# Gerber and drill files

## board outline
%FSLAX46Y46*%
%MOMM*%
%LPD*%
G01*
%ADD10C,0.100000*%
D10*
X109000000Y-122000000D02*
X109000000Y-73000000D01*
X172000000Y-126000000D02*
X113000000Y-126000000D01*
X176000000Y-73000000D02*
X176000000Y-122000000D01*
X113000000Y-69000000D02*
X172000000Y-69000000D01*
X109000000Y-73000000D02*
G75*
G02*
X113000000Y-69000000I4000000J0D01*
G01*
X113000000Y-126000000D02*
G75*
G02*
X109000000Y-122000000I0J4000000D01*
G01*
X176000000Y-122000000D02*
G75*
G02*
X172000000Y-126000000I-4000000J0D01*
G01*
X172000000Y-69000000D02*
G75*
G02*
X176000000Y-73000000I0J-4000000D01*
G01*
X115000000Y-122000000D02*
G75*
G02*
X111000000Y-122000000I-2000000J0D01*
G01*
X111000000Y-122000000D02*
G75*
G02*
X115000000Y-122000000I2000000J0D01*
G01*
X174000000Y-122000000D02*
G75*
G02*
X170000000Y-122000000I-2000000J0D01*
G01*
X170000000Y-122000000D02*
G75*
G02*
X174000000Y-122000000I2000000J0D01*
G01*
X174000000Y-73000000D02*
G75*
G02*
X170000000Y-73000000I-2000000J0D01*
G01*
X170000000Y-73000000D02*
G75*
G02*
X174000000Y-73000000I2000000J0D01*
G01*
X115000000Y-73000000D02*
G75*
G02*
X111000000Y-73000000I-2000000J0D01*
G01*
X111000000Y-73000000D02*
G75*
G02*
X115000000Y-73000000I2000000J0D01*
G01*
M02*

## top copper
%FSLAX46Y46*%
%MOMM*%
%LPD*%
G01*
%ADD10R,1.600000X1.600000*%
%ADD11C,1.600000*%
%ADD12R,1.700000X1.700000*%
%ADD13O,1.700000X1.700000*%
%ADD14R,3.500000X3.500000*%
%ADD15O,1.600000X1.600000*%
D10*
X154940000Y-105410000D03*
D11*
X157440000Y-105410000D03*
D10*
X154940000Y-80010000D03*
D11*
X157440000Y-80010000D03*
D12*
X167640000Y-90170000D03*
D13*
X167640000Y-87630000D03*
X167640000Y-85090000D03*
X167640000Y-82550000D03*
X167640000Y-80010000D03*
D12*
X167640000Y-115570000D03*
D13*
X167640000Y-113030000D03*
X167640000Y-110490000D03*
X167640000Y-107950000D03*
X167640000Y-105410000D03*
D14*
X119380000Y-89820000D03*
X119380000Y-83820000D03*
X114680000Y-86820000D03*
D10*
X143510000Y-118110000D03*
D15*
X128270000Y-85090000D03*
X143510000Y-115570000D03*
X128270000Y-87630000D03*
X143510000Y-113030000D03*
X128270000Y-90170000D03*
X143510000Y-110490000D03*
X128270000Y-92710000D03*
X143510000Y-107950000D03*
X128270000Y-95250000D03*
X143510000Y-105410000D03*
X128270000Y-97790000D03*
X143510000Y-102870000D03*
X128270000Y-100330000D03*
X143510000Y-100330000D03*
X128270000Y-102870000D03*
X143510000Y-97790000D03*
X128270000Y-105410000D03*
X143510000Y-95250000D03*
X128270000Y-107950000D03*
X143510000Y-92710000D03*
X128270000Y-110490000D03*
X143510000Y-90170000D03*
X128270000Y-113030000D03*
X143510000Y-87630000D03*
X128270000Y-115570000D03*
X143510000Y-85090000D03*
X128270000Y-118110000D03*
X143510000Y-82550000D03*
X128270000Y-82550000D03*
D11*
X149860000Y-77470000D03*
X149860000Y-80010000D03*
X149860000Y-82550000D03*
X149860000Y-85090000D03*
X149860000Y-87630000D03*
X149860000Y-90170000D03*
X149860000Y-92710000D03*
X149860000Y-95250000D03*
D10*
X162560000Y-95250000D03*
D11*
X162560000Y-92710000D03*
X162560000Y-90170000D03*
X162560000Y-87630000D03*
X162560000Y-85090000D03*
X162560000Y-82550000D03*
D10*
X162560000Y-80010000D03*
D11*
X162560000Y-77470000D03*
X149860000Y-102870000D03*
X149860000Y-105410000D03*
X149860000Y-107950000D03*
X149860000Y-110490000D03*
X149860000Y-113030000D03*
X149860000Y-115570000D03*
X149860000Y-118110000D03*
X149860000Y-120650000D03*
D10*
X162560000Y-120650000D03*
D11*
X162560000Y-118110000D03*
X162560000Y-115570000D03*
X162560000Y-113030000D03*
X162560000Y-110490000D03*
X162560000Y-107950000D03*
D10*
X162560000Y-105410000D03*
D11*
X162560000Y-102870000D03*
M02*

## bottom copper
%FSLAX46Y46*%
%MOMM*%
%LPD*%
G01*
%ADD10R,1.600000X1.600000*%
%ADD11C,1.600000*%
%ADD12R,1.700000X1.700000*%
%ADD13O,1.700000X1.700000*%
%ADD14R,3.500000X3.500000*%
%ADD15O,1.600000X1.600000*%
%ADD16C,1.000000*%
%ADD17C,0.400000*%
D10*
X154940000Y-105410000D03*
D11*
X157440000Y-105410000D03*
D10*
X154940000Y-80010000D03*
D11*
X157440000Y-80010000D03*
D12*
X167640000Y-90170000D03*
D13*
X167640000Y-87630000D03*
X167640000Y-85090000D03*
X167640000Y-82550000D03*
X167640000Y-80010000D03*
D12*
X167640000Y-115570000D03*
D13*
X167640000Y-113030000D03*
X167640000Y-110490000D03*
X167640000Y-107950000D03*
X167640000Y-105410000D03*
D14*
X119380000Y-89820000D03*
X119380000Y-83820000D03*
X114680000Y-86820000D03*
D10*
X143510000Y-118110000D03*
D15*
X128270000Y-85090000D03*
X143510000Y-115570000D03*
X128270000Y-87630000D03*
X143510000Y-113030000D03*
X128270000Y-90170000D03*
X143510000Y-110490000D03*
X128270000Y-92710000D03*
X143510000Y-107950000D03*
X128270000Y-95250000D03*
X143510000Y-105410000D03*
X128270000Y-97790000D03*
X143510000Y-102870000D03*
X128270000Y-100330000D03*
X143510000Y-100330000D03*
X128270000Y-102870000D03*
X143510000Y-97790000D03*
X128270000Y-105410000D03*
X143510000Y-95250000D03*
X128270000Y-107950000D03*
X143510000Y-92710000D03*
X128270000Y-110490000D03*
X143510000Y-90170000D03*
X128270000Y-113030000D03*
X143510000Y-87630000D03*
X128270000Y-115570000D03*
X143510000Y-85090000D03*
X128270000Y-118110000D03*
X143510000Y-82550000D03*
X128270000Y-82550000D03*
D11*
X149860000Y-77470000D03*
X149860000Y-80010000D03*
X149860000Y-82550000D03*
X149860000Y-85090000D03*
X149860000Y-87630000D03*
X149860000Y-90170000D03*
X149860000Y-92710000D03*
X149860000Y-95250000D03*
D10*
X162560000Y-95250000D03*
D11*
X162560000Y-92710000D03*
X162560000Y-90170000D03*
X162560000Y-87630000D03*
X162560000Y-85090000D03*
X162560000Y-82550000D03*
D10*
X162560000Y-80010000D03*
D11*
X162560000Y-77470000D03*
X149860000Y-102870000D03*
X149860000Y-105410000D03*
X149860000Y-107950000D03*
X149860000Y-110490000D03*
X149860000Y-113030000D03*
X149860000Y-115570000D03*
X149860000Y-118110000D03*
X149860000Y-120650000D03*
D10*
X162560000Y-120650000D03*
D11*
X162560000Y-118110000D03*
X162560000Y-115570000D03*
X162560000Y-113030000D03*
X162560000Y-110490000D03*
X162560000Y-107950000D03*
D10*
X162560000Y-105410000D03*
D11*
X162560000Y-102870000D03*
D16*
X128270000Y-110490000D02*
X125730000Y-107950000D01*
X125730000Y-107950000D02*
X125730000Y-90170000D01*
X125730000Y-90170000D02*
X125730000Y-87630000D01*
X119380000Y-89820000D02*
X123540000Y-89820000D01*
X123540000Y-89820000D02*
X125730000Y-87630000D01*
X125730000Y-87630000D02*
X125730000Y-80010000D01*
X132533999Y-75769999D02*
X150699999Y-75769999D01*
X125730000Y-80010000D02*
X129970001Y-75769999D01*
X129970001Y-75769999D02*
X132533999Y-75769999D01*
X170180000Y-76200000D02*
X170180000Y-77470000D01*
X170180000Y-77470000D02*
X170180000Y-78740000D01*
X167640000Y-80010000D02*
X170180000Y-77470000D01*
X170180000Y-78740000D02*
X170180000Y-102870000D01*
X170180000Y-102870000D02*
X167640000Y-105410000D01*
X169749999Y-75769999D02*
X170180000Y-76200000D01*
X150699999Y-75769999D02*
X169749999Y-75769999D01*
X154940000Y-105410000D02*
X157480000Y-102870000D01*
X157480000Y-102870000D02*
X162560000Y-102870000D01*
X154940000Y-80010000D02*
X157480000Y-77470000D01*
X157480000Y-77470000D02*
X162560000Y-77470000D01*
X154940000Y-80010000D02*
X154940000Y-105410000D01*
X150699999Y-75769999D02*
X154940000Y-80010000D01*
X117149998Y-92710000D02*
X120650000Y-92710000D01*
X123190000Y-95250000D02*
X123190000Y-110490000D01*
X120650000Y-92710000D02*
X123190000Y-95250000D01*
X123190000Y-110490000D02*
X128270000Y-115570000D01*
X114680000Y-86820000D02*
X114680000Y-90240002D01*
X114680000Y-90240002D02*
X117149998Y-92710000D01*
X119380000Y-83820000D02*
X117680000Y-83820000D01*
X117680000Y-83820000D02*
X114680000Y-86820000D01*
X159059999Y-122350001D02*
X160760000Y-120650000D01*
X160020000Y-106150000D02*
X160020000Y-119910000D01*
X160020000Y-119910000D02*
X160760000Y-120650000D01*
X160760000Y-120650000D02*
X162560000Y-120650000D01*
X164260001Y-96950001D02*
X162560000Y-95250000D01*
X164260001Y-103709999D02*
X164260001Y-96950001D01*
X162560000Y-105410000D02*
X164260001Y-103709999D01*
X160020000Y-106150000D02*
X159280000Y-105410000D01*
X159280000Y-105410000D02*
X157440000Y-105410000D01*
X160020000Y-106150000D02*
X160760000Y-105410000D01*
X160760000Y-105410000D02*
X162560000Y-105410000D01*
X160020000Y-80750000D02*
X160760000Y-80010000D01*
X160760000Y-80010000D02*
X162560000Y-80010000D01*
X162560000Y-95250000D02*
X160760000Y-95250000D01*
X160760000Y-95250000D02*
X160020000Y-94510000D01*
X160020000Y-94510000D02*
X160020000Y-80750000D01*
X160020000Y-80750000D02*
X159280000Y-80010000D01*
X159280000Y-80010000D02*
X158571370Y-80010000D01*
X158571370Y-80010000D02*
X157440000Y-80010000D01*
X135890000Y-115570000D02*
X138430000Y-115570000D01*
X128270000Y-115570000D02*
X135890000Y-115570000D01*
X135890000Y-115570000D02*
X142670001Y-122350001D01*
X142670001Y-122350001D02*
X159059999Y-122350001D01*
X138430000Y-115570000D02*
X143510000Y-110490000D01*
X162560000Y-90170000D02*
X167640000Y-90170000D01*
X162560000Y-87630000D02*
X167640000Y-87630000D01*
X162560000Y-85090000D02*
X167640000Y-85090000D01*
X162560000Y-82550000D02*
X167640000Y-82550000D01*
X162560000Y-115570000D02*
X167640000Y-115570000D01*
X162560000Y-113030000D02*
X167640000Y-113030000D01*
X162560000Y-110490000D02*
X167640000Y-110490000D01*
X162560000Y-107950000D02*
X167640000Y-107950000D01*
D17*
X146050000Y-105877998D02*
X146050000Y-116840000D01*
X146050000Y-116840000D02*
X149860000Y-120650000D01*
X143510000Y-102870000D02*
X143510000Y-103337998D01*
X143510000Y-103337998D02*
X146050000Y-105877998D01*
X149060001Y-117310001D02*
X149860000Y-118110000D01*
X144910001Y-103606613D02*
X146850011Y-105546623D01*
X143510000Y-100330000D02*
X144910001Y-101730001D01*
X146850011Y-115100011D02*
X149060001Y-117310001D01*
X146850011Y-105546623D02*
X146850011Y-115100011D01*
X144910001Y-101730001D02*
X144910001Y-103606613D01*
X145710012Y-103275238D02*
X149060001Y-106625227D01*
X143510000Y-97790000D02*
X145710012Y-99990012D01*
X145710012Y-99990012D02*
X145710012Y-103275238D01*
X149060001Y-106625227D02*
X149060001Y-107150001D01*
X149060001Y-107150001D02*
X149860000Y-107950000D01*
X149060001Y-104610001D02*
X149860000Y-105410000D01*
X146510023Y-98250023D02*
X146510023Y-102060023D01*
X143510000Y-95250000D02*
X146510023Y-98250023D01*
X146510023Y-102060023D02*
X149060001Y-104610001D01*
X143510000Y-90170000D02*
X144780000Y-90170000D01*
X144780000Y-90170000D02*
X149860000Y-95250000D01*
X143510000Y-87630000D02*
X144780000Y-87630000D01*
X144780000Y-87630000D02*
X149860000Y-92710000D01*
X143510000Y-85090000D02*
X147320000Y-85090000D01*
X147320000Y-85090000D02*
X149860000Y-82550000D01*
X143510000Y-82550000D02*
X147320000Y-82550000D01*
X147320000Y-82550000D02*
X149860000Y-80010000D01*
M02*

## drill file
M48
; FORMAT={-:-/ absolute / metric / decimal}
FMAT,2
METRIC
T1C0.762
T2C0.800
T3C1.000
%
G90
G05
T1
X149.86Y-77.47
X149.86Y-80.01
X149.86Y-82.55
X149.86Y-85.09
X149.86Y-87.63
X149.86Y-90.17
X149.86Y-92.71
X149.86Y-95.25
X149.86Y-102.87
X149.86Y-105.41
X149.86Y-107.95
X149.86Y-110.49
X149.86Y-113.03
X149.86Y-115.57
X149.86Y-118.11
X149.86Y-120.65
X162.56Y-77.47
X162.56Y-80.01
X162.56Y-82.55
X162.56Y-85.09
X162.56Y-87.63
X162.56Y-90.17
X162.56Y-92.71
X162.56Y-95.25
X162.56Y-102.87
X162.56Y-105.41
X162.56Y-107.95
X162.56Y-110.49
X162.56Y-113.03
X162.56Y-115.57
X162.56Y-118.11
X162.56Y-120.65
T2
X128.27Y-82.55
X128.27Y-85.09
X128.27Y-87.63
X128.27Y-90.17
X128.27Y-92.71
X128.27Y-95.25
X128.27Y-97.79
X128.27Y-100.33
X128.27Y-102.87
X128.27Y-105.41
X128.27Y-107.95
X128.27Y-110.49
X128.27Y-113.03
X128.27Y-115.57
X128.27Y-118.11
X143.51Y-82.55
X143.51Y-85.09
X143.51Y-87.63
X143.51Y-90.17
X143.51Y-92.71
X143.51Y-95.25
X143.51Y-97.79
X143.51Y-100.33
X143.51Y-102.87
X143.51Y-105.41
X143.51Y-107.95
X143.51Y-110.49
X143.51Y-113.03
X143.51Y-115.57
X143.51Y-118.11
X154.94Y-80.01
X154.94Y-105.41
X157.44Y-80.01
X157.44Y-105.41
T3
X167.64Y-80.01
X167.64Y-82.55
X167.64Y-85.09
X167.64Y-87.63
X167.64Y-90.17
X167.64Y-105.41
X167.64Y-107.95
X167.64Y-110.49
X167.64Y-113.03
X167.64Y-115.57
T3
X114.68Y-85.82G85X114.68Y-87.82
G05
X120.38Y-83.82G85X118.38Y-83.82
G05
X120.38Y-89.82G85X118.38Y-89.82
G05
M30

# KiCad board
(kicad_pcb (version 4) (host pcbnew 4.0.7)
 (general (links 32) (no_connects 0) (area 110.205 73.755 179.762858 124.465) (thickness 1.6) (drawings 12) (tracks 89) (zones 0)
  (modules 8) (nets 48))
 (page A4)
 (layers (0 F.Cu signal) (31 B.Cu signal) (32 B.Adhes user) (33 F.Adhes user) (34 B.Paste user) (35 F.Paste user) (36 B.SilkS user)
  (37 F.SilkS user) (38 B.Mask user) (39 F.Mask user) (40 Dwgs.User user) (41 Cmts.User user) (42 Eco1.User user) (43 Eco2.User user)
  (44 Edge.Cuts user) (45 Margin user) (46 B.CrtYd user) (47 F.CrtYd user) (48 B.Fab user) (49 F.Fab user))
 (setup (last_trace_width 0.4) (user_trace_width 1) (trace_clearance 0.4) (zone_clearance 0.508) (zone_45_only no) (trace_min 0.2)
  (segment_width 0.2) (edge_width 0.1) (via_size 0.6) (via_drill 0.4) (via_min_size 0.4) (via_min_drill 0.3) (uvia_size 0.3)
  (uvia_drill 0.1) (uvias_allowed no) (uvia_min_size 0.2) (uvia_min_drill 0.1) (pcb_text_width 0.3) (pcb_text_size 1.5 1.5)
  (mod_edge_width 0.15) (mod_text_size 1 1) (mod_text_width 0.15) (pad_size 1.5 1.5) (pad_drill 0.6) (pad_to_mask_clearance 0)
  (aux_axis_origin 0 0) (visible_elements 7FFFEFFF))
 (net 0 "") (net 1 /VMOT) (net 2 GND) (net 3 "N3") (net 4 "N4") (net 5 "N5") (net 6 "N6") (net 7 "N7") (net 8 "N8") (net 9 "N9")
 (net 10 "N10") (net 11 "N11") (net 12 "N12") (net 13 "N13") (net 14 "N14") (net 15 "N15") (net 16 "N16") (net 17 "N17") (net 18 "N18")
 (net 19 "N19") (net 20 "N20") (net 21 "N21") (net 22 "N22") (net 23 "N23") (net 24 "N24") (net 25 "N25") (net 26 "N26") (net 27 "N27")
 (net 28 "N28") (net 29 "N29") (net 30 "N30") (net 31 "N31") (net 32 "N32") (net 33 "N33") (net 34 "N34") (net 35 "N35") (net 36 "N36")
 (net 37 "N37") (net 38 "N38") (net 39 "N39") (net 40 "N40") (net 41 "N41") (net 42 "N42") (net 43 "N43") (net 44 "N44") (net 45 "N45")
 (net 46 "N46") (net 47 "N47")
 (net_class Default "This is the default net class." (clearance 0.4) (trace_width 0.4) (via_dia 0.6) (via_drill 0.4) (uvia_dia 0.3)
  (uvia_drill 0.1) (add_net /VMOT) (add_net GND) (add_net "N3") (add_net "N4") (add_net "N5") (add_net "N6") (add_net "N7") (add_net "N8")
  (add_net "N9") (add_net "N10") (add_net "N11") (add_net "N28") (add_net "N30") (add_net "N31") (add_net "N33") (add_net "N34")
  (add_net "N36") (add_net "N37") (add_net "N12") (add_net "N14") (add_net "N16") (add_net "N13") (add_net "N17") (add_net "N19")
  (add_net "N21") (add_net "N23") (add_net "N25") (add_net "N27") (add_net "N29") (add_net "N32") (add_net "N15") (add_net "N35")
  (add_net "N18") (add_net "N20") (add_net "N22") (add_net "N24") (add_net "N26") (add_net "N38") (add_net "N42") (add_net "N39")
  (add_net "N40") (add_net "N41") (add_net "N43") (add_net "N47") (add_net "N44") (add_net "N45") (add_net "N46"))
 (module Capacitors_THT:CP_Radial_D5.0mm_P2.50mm (layer F.Cu) (at 154.94 105.41)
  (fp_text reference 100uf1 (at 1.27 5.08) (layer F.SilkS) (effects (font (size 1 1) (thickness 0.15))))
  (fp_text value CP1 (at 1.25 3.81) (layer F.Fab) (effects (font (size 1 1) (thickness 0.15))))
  (pad 1 thru_hole rect (at 0 0) (size 1.6 1.6) (drill 0.8) (layers *.Cu *.Mask) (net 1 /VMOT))
  (pad 2 thru_hole circle (at 2.5 0) (size 1.6 1.6) (drill 0.8) (layers *.Cu *.Mask) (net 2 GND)))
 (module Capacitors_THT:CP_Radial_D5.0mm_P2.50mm (layer F.Cu) (at 154.94 80.01)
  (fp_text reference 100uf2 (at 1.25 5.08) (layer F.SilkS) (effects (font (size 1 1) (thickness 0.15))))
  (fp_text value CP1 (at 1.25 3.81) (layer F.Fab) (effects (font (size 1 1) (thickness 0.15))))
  (pad 1 thru_hole rect (at 0 0) (size 1.6 1.6) (drill 0.8) (layers *.Cu *.Mask) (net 1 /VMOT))
  (pad 2 thru_hole circle (at 2.5 0) (size 1.6 1.6) (drill 0.8) (layers *.Cu *.Mask) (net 2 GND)))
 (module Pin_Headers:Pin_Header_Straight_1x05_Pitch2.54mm (layer F.Cu) (at 167.64 90.17 180)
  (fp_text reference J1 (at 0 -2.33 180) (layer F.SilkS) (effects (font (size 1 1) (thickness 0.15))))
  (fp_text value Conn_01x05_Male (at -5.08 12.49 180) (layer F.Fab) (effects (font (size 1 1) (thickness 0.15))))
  (pad 1 thru_hole rect (at 0 0 180) (size 1.7 1.7) (drill 1) (layers *.Cu *.Mask) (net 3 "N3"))
  (pad 2 thru_hole oval (at 0 2.54 180) (size 1.7 1.7) (drill 1) (layers *.Cu *.Mask) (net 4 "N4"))
  (pad 3 thru_hole oval (at 0 5.08 180) (size 1.7 1.7) (drill 1) (layers *.Cu *.Mask) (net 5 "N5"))
  (pad 4 thru_hole oval (at 0 7.62 180) (size 1.7 1.7) (drill 1) (layers *.Cu *.Mask) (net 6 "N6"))
  (pad 5 thru_hole oval (at 0 10.16 180) (size 1.7 1.7) (drill 1) (layers *.Cu *.Mask) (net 1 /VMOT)))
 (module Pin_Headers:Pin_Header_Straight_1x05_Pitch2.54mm (layer F.Cu) (at 167.64 115.57 180)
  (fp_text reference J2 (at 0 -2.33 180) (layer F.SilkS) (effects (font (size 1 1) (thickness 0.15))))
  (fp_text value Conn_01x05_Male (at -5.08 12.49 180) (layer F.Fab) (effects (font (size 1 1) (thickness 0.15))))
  (pad 1 thru_hole rect (at 0 0 180) (size 1.7 1.7) (drill 1) (layers *.Cu *.Mask) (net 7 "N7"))
  (pad 2 thru_hole oval (at 0 2.54 180) (size 1.7 1.7) (drill 1) (layers *.Cu *.Mask) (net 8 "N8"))
  (pad 3 thru_hole oval (at 0 5.08 180) (size 1.7 1.7) (drill 1) (layers *.Cu *.Mask) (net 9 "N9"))
  (pad 4 thru_hole oval (at 0 7.62 180) (size 1.7 1.7) (drill 1) (layers *.Cu *.Mask) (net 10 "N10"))
  (pad 5 thru_hole oval (at 0 10.16 180) (size 1.7 1.7) (drill 1) (layers *.Cu *.Mask) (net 1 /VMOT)))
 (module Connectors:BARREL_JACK (layer F.Cu) (at 119.38 89.82 270)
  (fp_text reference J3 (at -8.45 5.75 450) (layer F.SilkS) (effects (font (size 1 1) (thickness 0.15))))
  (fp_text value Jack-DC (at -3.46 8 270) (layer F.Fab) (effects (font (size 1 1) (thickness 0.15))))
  (pad 1 thru_hole rect (at 0 0 270) (size 3.5 3.5) (drill oval 1 3) (layers *.Cu *.Mask) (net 1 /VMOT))
  (pad 2 thru_hole rect (at -6 0 270) (size 3.5 3.5) (drill oval 1 3) (layers *.Cu *.Mask) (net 2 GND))
  (pad 3 thru_hole rect (at -3 4.7 270) (size 3.5 3.5) (drill oval 3 1) (layers *.Cu *.Mask) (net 2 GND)))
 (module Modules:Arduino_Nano (layer F.Cu) (at 143.51 118.11 180)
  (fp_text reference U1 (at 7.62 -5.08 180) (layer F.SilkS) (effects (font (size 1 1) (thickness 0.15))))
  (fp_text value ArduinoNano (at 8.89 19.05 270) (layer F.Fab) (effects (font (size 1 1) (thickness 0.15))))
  (pad 1 thru_hole rect (at 0 0 180) (size 1.6 1.6) (drill 0.8) (layers *.Cu *.Mask) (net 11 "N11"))
  (pad 17 thru_hole oval (at 15.24 33.02 180) (size 1.6 1.6) (drill 0.8) (layers *.Cu *.Mask) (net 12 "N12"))
  (pad 2 thru_hole oval (at 0 2.54 180) (size 1.6 1.6) (drill 0.8) (layers *.Cu *.Mask) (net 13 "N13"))
  (pad 18 thru_hole oval (at 15.24 30.48 180) (size 1.6 1.6) (drill 0.8) (layers *.Cu *.Mask) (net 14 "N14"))
  (pad 3 thru_hole oval (at 0 5.08 180) (size 1.6 1.6) (drill 0.8) (layers *.Cu *.Mask) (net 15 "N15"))
  (pad 19 thru_hole oval (at 15.24 27.94 180) (size 1.6 1.6) (drill 0.8) (layers *.Cu *.Mask) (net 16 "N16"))
  (pad 4 thru_hole oval (at 0 7.62 180) (size 1.6 1.6) (drill 0.8) (layers *.Cu *.Mask) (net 2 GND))
  (pad 20 thru_hole oval (at 15.24 25.4 180) (size 1.6 1.6) (drill 0.8) (layers *.Cu *.Mask) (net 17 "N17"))
  (pad 5 thru_hole oval (at 0 10.16 180) (size 1.6 1.6) (drill 0.8) (layers *.Cu *.Mask) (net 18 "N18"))
  (pad 21 thru_hole oval (at 15.24 22.86 180) (size 1.6 1.6) (drill 0.8) (layers *.Cu *.Mask) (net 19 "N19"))
  (pad 6 thru_hole oval (at 0 12.7 180) (size 1.6 1.6) (drill 0.8) (layers *.Cu *.Mask) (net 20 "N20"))
  (pad 22 thru_hole oval (at 15.24 20.32 180) (size 1.6 1.6) (drill 0.8) (layers *.Cu *.Mask) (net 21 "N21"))
  (pad 7 thru_hole oval (at 0 15.24 180) (size 1.6 1.6) (drill 0.8) (layers *.Cu *.Mask) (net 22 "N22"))
  (pad 23 thru_hole oval (at 15.24 17.78 180) (size 1.6 1.6) (drill 0.8) (layers *.Cu *.Mask) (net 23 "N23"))
  (pad 8 thru_hole oval (at 0 17.78 180) (size 1.6 1.6) (drill 0.8) (layers *.Cu *.Mask) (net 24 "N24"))
  (pad 24 thru_hole oval (at 15.24 15.24 180) (size 1.6 1.6) (drill 0.8) (layers *.Cu *.Mask) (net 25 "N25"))
  (pad 9 thru_hole oval (at 0 20.32 180) (size 1.6 1.6) (drill 0.8) (layers *.Cu *.Mask) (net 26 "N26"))
  (pad 25 thru_hole oval (at 15.24 12.7 180) (size 1.6 1.6) (drill 0.8) (layers *.Cu *.Mask) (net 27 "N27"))
  (pad 10 thru_hole oval (at 0 22.86 180) (size 1.6 1.6) (drill 0.8) (layers *.Cu *.Mask) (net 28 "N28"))
  (pad 26 thru_hole oval (at 15.24 10.16 180) (size 1.6 1.6) (drill 0.8) (layers *.Cu *.Mask) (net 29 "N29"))
  (pad 11 thru_hole oval (at 0 25.4 180) (size 1.6 1.6) (drill 0.8) (layers *.Cu *.Mask) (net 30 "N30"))
  (pad 27 thru_hole oval (at 15.24 7.62 180) (size 1.6 1.6) (drill 0.8) (layers *.Cu *.Mask) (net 1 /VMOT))
  (pad 12 thru_hole oval (at 0 27.94 180) (size 1.6 1.6) (drill 0.8) (layers *.Cu *.Mask) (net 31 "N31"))
  (pad 28 thru_hole oval (at 15.24 5.08 180) (size 1.6 1.6) (drill 0.8) (layers *.Cu *.Mask) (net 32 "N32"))
  (pad 13 thru_hole oval (at 0 30.48 180) (size 1.6 1.6) (drill 0.8) (layers *.Cu *.Mask) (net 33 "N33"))
  (pad 29 thru_hole oval (at 15.24 2.54 180) (size 1.6 1.6) (drill 0.8) (layers *.Cu *.Mask) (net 2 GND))
  (pad 14 thru_hole oval (at 0 33.02 180) (size 1.6 1.6) (drill 0.8) (layers *.Cu *.Mask) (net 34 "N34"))
  (pad 30 thru_hole oval (at 15.24 0 180) (size 1.6 1.6) (drill 0.8) (layers *.Cu *.Mask) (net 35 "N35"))
  (pad 15 thru_hole oval (at 0 35.56 180) (size 1.6 1.6) (drill 0.8) (layers *.Cu *.Mask) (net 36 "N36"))
  (pad 16 thru_hole oval (at 15.24 35.56 180) (size 1.6 1.6) (drill 0.8) (layers *.Cu *.Mask) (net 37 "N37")))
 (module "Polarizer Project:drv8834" (layer F.Cu) (at 149.86 77.47)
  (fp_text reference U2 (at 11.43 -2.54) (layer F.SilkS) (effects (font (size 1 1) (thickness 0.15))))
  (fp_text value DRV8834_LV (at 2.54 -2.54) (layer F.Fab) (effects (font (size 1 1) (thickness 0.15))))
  (pad 1 thru_hole circle (at 0 0) (size 1.6 1.6) (drill 0.762) (layers *.Cu *.Mask) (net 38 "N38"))
  (pad 2 thru_hole circle (at 0 2.54) (size 1.6 1.6) (drill 0.762) (layers *.Cu *.Mask) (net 36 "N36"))
  (pad 3 thru_hole circle (at 0 5.08) (size 1.6 1.6) (drill 0.762) (layers *.Cu *.Mask) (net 34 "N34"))
  (pad 4 thru_hole circle (at 0 7.62) (size 1.6 1.6) (drill 0.762) (layers *.Cu *.Mask) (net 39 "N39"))
  (pad 5 thru_hole circle (at 0 10.16) (size 1.6 1.6) (drill 0.762) (layers *.Cu *.Mask) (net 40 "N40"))
  (pad 6 thru_hole circle (at 0 12.7) (size 1.6 1.6) (drill 0.762) (layers *.Cu *.Mask) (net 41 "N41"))
  (pad 7 thru_hole circle (at 0 15.24) (size 1.6 1.6) (drill 0.762) (layers *.Cu *.Mask) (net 33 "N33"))
  (pad 8 thru_hole circle (at 0 17.78) (size 1.6 1.6) (drill 0.762) (layers *.Cu *.Mask) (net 31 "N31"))
  (pad 9 thru_hole rect (at 12.7 17.78) (size 1.6 1.6) (drill 0.762) (layers *.Cu *.Mask) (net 2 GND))
  (pad 10 thru_hole circle (at 12.7 15.24) (size 1.6 1.6) (drill 0.762) (layers *.Cu *.Mask) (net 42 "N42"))
  (pad 11 thru_hole circle (at 12.7 12.7) (size 1.6 1.6) (drill 0.762) (layers *.Cu *.Mask) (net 3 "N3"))
  (pad 12 thru_hole circle (at 12.7 10.16) (size 1.6 1.6) (drill 0.762) (layers *.Cu *.Mask) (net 4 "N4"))
  (pad 13 thru_hole circle (at 12.7 7.62) (size 1.6 1.6) (drill 0.762) (layers *.Cu *.Mask) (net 5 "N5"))
  (pad 14 thru_hole circle (at 12.7 5.08) (size 1.6 1.6) (drill 0.762) (layers *.Cu *.Mask) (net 6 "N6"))
  (pad 15 thru_hole rect (at 12.7 2.54) (size 1.6 1.6) (drill 0.762) (layers *.Cu *.Mask) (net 2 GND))
  (pad 16 thru_hole circle (at 12.7 0) (size 1.6 1.6) (drill 0.762) (layers *.Cu *.Mask) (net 1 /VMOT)))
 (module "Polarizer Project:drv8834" (layer F.Cu) (at 149.86 102.87)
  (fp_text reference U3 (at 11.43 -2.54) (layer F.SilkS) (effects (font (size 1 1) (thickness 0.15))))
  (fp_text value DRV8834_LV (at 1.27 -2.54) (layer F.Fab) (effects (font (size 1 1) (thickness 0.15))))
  (pad 1 thru_hole circle (at 0 0) (size 1.6 1.6) (drill 0.762) (layers *.Cu *.Mask) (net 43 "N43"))
  (pad 2 thru_hole circle (at 0 2.54) (size 1.6 1.6) (drill 0.762) (layers *.Cu *.Mask) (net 28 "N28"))
  (pad 3 thru_hole circle (at 0 5.08) (size 1.6 1.6) (drill 0.762) (layers *.Cu *.Mask) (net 26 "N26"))
  (pad 4 thru_hole circle (at 0 7.62) (size 1.6 1.6) (drill 0.762) (layers *.Cu *.Mask) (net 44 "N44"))
  (pad 5 thru_hole circle (at 0 10.16) (size 1.6 1.6) (drill 0.762) (layers *.Cu *.Mask) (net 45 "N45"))
  (pad 6 thru_hole circle (at 0 12.7) (size 1.6 1.6) (drill 0.762) (layers *.Cu *.Mask) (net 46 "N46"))
  (pad 7 thru_hole circle (at 0 15.24) (size 1.6 1.6) (drill 0.762) (layers *.Cu *.Mask) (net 24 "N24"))
  (pad 8 thru_hole circle (at 0 17.78) (size 1.6 1.6) (drill 0.762) (layers *.Cu *.Mask) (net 22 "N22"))
  (pad 9 thru_hole rect (at 12.7 17.78) (size 1.6 1.6) (drill 0.762) (layers *.Cu *.Mask) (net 2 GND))
  (pad 10 thru_hole circle (at 12.7 15.24) (size 1.6 1.6) (drill 0.762) (layers *.Cu *.Mask) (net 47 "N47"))
  (pad 11 thru_hole circle (at 12.7 12.7) (size 1.6 1.6) (drill 0.762) (layers *.Cu *.Mask) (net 7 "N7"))
  (pad 12 thru_hole circle (at 12.7 10.16) (size 1.6 1.6) (drill 0.762) (layers *.Cu *.Mask) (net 8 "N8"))
  (pad 13 thru_hole circle (at 12.7 7.62) (size 1.6 1.6) (drill 0.762) (layers *.Cu *.Mask) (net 9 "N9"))
  (pad 14 thru_hole circle (at 12.7 5.08) (size 1.6 1.6) (drill 0.762) (layers *.Cu *.Mask) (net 10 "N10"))
  (pad 15 thru_hole rect (at 12.7 2.54) (size 1.6 1.6) (drill 0.762) (layers *.Cu *.Mask) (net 2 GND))
  (pad 16 thru_hole circle (at 12.7 0) (size 1.6 1.6) (drill 0.762) (layers *.Cu *.Mask) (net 1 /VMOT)))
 (gr_line (start 109 122) (end 109 73) (layer Edge.Cuts) (width 0.1))
 (gr_line (start 172 126) (end 113 126) (layer Edge.Cuts) (width 0.1))
 (gr_line (start 176 73) (end 176 122) (layer Edge.Cuts) (width 0.1))
 (gr_line (start 113 69) (end 172 69) (layer Edge.Cuts) (width 0.1))
 (gr_arc (start 113 73) (end 109 73) (angle 90) (layer Edge.Cuts) (width 0.1))
 (gr_arc (start 113 122) (end 113 126) (angle 90) (layer Edge.Cuts) (width 0.1))
 (gr_arc (start 172 122) (end 176 122) (angle 90) (layer Edge.Cuts) (width 0.1))
 (gr_arc (start 172 73) (end 172 69) (angle 90) (layer Edge.Cuts) (width 0.1))
 (gr_circle (center 113 122) (end 115 122) (layer Edge.Cuts) (width 0.1))
 (gr_circle (center 172 122) (end 174 122) (layer Edge.Cuts) (width 0.1))
 (gr_circle (center 172 73) (end 174 73) (layer Edge.Cuts) (width 0.1))
 (gr_circle (center 113 73) (end 115 73) (layer Edge.Cuts) (width 0.1))
 (segment (start 128.27 110.49) (end 125.73 107.95) (width 1) (layer B.Cu) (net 1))
 (segment (start 125.73 107.95) (end 125.73 90.17) (width 1) (layer B.Cu) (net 1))
 (segment (start 125.73 90.17) (end 125.73 87.63) (width 1) (layer B.Cu) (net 1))
 (segment (start 119.38 89.82) (end 123.54 89.82) (width 1) (layer B.Cu) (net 1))
 (segment (start 123.54 89.82) (end 125.73 87.63) (width 1) (layer B.Cu) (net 1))
 (segment (start 125.73 87.63) (end 125.73 80.01) (width 1) (layer B.Cu) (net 1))
 (segment (start 132.533999 75.769999) (end 150.699999 75.769999) (width 1) (layer B.Cu) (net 1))
 (segment (start 125.73 80.01) (end 129.970001 75.769999) (width 1) (layer B.Cu) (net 1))
 (segment (start 129.970001 75.769999) (end 132.533999 75.769999) (width 1) (layer B.Cu) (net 1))
 (segment (start 170.18 76.2) (end 170.18 77.47) (width 1) (layer B.Cu) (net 1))
 (segment (start 170.18 77.47) (end 170.18 78.74) (width 1) (layer B.Cu) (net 1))
 (segment (start 167.64 80.01) (end 170.18 77.47) (width 1) (layer B.Cu) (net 1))
 (segment (start 170.18 78.74) (end 170.18 102.87) (width 1) (layer B.Cu) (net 1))
 (segment (start 170.18 102.87) (end 167.64 105.41) (width 1) (layer B.Cu) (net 1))
 (segment (start 169.749999 75.769999) (end 170.18 76.2) (width 1) (layer B.Cu) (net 1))
 (segment (start 150.699999 75.769999) (end 169.749999 75.769999) (width 1) (layer B.Cu) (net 1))
 (segment (start 154.94 105.41) (end 157.48 102.87) (width 1) (layer B.Cu) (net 1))
 (segment (start 157.48 102.87) (end 162.56 102.87) (width 1) (layer B.Cu) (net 1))
 (segment (start 154.94 80.01) (end 157.48 77.47) (width 1) (layer B.Cu) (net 1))
 (segment (start 157.48 77.47) (end 162.56 77.47) (width 1) (layer B.Cu) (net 1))
 (segment (start 154.94 80.01) (end 154.94 105.41) (width 1) (layer B.Cu) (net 1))
 (segment (start 150.699999 75.769999) (end 154.94 80.01) (width 1) (layer B.Cu) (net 1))
 (segment (start 117.149998 92.71) (end 120.65 92.71) (width 1) (layer B.Cu) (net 2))
 (segment (start 123.19 95.25) (end 123.19 110.49) (width 1) (layer B.Cu) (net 2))
 (segment (start 120.65 92.71) (end 123.19 95.25) (width 1) (layer B.Cu) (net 2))
 (segment (start 123.19 110.49) (end 128.27 115.57) (width 1) (layer B.Cu) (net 2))
 (segment (start 114.68 86.82) (end 114.68 90.240002) (width 1) (layer B.Cu) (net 2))
 (segment (start 114.68 90.240002) (end 117.149998 92.71) (width 1) (layer B.Cu) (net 2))
 (segment (start 119.38 83.82) (end 117.68 83.82) (width 1) (layer B.Cu) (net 2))
 (segment (start 117.68 83.82) (end 114.68 86.82) (width 1) (layer B.Cu) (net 2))
 (segment (start 159.059999 122.350001) (end 160.76 120.65) (width 1) (layer B.Cu) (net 2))
 (segment (start 160.02 106.15) (end 160.02 119.91) (width 1) (layer B.Cu) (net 2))
 (segment (start 160.02 119.91) (end 160.76 120.65) (width 1) (layer B.Cu) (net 2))
 (segment (start 160.76 120.65) (end 162.56 120.65) (width 1) (layer B.Cu) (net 2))
 (segment (start 164.260001 96.950001) (end 162.56 95.25) (width 1) (layer B.Cu) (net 2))
 (segment (start 164.260001 103.709999) (end 164.260001 96.950001) (width 1) (layer B.Cu) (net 2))
 (segment (start 162.56 105.41) (end 164.260001 103.709999) (width 1) (layer B.Cu) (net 2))
 (segment (start 160.02 106.15) (end 159.28 105.41) (width 1) (layer B.Cu) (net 2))
 (segment (start 159.28 105.41) (end 157.44 105.41) (width 1) (layer B.Cu) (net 2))
 (segment (start 160.02 106.15) (end 160.76 105.41) (width 1) (layer B.Cu) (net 2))
 (segment (start 160.76 105.41) (end 162.56 105.41) (width 1) (layer B.Cu) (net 2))
 (segment (start 160.02 80.75) (end 160.76 80.01) (width 1) (layer B.Cu) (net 2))
 (segment (start 160.76 80.01) (end 162.56 80.01) (width 1) (layer B.Cu) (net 2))
 (segment (start 162.56 95.25) (end 160.76 95.25) (width 1) (layer B.Cu) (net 2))
 (segment (start 160.76 95.25) (end 160.02 94.51) (width 1) (layer B.Cu) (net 2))
 (segment (start 160.02 94.51) (end 160.02 80.75) (width 1) (layer B.Cu) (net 2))
 (segment (start 160.02 80.75) (end 159.28 80.01) (width 1) (layer B.Cu) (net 2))
 (segment (start 159.28 80.01) (end 158.57137 80.01) (width 1) (layer B.Cu) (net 2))
 (segment (start 158.57137 80.01) (end 157.44 80.01) (width 1) (layer B.Cu) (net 2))
 (segment (start 135.89 115.57) (end 138.43 115.57) (width 1) (layer B.Cu) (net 2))
 (segment (start 128.27 115.57) (end 135.89 115.57) (width 1) (layer B.Cu) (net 2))
 (segment (start 135.89 115.57) (end 142.670001 122.350001) (width 1) (layer B.Cu) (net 2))
 (segment (start 142.670001 122.350001) (end 159.059999 122.350001) (width 1) (layer B.Cu) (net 2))
 (segment (start 138.43 115.57) (end 143.51 110.49) (width 1) (layer B.Cu) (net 2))
 (segment (start 162.56 90.17) (end 167.64 90.17) (width 1) (layer B.Cu) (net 3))
 (segment (start 162.56 87.63) (end 167.64 87.63) (width 1) (layer B.Cu) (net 4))
 (segment (start 162.56 85.09) (end 167.64 85.09) (width 1) (layer B.Cu) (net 5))
 (segment (start 162.56 82.55) (end 167.64 82.55) (width 1) (layer B.Cu) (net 6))
 (segment (start 162.56 115.57) (end 167.64 115.57) (width 1) (layer B.Cu) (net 7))
 (segment (start 162.56 113.03) (end 167.64 113.03) (width 1) (layer B.Cu) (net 8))
 (segment (start 162.56 110.49) (end 167.64 110.49) (width 1) (layer B.Cu) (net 9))
 (segment (start 162.56 107.95) (end 167.64 107.95) (width 1) (layer B.Cu) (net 10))
 (segment (start 146.05 105.877998) (end 146.05 116.84) (width 0.4) (layer B.Cu) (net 22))
 (segment (start 146.05 116.84) (end 149.86 120.65) (width 0.4) (layer B.Cu) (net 22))
 (segment (start 143.51 102.87) (end 143.51 103.337998) (width 0.4) (layer B.Cu) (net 22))
 (segment (start 143.51 103.337998) (end 146.05 105.877998) (width 0.4) (layer B.Cu) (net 22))
 (segment (start 149.060001 117.310001) (end 149.86 118.11) (width 0.4) (layer B.Cu) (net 24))
 (segment (start 144.910001 103.606613) (end 146.850011 105.546623) (width 0.4) (layer B.Cu) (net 24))
 (segment (start 143.51 100.33) (end 144.910001 101.730001) (width 0.4) (layer B.Cu) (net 24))
 (segment (start 146.850011 115.100011) (end 149.060001 117.310001) (width 0.4) (layer B.Cu) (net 24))
 (segment (start 146.850011 105.546623) (end 146.850011 115.100011) (width 0.4) (layer B.Cu) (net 24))
 (segment (start 144.910001 101.730001) (end 144.910001 103.606613) (width 0.4) (layer B.Cu) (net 24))
 (segment (start 145.710012 103.275238) (end 149.060001 106.625227) (width 0.4) (layer B.Cu) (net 26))
 (segment (start 143.51 97.79) (end 145.710012 99.990012) (width 0.4) (layer B.Cu) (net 26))
 (segment (start 145.710012 99.990012) (end 145.710012 103.275238) (width 0.4) (layer B.Cu) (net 26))
 (segment (start 149.060001 106.625227) (end 149.060001 107.150001) (width 0.4) (layer B.Cu) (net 26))
 (segment (start 149.060001 107.150001) (end 149.86 107.95) (width 0.4) (layer B.Cu) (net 26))
 (segment (start 149.060001 104.610001) (end 149.86 105.41) (width 0.4) (layer B.Cu) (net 28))
 (segment (start 146.510023 98.250023) (end 146.510023 102.060023) (width 0.4) (layer B.Cu) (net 28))
 (segment (start 143.51 95.25) (end 146.510023 98.250023) (width 0.4) (layer B.Cu) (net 28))
 (segment (start 146.510023 102.060023) (end 149.060001 104.610001) (width 0.4) (layer B.Cu) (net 28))
 (segment (start 143.51 90.17) (end 144.78 90.17) (width 0.4) (layer B.Cu) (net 31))
 (segment (start 144.78 90.17) (end 149.86 95.25) (width 0.4) (layer B.Cu) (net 31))
 (segment (start 143.51 87.63) (end 144.78 87.63) (width 0.4) (layer B.Cu) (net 33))
 (segment (start 144.78 87.63) (end 149.86 92.71) (width 0.4) (layer B.Cu) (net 33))
 (segment (start 143.51 85.09) (end 147.32 85.09) (width 0.4) (layer B.Cu) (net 34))
 (segment (start 147.32 85.09) (end 149.86 82.55) (width 0.4) (layer B.Cu) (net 34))
 (segment (start 143.51 82.55) (end 147.32 82.55) (width 0.4) (layer B.Cu) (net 36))
 (segment (start 147.32 82.55) (end 149.86 80.01) (width 0.4) (layer B.Cu) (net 36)))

